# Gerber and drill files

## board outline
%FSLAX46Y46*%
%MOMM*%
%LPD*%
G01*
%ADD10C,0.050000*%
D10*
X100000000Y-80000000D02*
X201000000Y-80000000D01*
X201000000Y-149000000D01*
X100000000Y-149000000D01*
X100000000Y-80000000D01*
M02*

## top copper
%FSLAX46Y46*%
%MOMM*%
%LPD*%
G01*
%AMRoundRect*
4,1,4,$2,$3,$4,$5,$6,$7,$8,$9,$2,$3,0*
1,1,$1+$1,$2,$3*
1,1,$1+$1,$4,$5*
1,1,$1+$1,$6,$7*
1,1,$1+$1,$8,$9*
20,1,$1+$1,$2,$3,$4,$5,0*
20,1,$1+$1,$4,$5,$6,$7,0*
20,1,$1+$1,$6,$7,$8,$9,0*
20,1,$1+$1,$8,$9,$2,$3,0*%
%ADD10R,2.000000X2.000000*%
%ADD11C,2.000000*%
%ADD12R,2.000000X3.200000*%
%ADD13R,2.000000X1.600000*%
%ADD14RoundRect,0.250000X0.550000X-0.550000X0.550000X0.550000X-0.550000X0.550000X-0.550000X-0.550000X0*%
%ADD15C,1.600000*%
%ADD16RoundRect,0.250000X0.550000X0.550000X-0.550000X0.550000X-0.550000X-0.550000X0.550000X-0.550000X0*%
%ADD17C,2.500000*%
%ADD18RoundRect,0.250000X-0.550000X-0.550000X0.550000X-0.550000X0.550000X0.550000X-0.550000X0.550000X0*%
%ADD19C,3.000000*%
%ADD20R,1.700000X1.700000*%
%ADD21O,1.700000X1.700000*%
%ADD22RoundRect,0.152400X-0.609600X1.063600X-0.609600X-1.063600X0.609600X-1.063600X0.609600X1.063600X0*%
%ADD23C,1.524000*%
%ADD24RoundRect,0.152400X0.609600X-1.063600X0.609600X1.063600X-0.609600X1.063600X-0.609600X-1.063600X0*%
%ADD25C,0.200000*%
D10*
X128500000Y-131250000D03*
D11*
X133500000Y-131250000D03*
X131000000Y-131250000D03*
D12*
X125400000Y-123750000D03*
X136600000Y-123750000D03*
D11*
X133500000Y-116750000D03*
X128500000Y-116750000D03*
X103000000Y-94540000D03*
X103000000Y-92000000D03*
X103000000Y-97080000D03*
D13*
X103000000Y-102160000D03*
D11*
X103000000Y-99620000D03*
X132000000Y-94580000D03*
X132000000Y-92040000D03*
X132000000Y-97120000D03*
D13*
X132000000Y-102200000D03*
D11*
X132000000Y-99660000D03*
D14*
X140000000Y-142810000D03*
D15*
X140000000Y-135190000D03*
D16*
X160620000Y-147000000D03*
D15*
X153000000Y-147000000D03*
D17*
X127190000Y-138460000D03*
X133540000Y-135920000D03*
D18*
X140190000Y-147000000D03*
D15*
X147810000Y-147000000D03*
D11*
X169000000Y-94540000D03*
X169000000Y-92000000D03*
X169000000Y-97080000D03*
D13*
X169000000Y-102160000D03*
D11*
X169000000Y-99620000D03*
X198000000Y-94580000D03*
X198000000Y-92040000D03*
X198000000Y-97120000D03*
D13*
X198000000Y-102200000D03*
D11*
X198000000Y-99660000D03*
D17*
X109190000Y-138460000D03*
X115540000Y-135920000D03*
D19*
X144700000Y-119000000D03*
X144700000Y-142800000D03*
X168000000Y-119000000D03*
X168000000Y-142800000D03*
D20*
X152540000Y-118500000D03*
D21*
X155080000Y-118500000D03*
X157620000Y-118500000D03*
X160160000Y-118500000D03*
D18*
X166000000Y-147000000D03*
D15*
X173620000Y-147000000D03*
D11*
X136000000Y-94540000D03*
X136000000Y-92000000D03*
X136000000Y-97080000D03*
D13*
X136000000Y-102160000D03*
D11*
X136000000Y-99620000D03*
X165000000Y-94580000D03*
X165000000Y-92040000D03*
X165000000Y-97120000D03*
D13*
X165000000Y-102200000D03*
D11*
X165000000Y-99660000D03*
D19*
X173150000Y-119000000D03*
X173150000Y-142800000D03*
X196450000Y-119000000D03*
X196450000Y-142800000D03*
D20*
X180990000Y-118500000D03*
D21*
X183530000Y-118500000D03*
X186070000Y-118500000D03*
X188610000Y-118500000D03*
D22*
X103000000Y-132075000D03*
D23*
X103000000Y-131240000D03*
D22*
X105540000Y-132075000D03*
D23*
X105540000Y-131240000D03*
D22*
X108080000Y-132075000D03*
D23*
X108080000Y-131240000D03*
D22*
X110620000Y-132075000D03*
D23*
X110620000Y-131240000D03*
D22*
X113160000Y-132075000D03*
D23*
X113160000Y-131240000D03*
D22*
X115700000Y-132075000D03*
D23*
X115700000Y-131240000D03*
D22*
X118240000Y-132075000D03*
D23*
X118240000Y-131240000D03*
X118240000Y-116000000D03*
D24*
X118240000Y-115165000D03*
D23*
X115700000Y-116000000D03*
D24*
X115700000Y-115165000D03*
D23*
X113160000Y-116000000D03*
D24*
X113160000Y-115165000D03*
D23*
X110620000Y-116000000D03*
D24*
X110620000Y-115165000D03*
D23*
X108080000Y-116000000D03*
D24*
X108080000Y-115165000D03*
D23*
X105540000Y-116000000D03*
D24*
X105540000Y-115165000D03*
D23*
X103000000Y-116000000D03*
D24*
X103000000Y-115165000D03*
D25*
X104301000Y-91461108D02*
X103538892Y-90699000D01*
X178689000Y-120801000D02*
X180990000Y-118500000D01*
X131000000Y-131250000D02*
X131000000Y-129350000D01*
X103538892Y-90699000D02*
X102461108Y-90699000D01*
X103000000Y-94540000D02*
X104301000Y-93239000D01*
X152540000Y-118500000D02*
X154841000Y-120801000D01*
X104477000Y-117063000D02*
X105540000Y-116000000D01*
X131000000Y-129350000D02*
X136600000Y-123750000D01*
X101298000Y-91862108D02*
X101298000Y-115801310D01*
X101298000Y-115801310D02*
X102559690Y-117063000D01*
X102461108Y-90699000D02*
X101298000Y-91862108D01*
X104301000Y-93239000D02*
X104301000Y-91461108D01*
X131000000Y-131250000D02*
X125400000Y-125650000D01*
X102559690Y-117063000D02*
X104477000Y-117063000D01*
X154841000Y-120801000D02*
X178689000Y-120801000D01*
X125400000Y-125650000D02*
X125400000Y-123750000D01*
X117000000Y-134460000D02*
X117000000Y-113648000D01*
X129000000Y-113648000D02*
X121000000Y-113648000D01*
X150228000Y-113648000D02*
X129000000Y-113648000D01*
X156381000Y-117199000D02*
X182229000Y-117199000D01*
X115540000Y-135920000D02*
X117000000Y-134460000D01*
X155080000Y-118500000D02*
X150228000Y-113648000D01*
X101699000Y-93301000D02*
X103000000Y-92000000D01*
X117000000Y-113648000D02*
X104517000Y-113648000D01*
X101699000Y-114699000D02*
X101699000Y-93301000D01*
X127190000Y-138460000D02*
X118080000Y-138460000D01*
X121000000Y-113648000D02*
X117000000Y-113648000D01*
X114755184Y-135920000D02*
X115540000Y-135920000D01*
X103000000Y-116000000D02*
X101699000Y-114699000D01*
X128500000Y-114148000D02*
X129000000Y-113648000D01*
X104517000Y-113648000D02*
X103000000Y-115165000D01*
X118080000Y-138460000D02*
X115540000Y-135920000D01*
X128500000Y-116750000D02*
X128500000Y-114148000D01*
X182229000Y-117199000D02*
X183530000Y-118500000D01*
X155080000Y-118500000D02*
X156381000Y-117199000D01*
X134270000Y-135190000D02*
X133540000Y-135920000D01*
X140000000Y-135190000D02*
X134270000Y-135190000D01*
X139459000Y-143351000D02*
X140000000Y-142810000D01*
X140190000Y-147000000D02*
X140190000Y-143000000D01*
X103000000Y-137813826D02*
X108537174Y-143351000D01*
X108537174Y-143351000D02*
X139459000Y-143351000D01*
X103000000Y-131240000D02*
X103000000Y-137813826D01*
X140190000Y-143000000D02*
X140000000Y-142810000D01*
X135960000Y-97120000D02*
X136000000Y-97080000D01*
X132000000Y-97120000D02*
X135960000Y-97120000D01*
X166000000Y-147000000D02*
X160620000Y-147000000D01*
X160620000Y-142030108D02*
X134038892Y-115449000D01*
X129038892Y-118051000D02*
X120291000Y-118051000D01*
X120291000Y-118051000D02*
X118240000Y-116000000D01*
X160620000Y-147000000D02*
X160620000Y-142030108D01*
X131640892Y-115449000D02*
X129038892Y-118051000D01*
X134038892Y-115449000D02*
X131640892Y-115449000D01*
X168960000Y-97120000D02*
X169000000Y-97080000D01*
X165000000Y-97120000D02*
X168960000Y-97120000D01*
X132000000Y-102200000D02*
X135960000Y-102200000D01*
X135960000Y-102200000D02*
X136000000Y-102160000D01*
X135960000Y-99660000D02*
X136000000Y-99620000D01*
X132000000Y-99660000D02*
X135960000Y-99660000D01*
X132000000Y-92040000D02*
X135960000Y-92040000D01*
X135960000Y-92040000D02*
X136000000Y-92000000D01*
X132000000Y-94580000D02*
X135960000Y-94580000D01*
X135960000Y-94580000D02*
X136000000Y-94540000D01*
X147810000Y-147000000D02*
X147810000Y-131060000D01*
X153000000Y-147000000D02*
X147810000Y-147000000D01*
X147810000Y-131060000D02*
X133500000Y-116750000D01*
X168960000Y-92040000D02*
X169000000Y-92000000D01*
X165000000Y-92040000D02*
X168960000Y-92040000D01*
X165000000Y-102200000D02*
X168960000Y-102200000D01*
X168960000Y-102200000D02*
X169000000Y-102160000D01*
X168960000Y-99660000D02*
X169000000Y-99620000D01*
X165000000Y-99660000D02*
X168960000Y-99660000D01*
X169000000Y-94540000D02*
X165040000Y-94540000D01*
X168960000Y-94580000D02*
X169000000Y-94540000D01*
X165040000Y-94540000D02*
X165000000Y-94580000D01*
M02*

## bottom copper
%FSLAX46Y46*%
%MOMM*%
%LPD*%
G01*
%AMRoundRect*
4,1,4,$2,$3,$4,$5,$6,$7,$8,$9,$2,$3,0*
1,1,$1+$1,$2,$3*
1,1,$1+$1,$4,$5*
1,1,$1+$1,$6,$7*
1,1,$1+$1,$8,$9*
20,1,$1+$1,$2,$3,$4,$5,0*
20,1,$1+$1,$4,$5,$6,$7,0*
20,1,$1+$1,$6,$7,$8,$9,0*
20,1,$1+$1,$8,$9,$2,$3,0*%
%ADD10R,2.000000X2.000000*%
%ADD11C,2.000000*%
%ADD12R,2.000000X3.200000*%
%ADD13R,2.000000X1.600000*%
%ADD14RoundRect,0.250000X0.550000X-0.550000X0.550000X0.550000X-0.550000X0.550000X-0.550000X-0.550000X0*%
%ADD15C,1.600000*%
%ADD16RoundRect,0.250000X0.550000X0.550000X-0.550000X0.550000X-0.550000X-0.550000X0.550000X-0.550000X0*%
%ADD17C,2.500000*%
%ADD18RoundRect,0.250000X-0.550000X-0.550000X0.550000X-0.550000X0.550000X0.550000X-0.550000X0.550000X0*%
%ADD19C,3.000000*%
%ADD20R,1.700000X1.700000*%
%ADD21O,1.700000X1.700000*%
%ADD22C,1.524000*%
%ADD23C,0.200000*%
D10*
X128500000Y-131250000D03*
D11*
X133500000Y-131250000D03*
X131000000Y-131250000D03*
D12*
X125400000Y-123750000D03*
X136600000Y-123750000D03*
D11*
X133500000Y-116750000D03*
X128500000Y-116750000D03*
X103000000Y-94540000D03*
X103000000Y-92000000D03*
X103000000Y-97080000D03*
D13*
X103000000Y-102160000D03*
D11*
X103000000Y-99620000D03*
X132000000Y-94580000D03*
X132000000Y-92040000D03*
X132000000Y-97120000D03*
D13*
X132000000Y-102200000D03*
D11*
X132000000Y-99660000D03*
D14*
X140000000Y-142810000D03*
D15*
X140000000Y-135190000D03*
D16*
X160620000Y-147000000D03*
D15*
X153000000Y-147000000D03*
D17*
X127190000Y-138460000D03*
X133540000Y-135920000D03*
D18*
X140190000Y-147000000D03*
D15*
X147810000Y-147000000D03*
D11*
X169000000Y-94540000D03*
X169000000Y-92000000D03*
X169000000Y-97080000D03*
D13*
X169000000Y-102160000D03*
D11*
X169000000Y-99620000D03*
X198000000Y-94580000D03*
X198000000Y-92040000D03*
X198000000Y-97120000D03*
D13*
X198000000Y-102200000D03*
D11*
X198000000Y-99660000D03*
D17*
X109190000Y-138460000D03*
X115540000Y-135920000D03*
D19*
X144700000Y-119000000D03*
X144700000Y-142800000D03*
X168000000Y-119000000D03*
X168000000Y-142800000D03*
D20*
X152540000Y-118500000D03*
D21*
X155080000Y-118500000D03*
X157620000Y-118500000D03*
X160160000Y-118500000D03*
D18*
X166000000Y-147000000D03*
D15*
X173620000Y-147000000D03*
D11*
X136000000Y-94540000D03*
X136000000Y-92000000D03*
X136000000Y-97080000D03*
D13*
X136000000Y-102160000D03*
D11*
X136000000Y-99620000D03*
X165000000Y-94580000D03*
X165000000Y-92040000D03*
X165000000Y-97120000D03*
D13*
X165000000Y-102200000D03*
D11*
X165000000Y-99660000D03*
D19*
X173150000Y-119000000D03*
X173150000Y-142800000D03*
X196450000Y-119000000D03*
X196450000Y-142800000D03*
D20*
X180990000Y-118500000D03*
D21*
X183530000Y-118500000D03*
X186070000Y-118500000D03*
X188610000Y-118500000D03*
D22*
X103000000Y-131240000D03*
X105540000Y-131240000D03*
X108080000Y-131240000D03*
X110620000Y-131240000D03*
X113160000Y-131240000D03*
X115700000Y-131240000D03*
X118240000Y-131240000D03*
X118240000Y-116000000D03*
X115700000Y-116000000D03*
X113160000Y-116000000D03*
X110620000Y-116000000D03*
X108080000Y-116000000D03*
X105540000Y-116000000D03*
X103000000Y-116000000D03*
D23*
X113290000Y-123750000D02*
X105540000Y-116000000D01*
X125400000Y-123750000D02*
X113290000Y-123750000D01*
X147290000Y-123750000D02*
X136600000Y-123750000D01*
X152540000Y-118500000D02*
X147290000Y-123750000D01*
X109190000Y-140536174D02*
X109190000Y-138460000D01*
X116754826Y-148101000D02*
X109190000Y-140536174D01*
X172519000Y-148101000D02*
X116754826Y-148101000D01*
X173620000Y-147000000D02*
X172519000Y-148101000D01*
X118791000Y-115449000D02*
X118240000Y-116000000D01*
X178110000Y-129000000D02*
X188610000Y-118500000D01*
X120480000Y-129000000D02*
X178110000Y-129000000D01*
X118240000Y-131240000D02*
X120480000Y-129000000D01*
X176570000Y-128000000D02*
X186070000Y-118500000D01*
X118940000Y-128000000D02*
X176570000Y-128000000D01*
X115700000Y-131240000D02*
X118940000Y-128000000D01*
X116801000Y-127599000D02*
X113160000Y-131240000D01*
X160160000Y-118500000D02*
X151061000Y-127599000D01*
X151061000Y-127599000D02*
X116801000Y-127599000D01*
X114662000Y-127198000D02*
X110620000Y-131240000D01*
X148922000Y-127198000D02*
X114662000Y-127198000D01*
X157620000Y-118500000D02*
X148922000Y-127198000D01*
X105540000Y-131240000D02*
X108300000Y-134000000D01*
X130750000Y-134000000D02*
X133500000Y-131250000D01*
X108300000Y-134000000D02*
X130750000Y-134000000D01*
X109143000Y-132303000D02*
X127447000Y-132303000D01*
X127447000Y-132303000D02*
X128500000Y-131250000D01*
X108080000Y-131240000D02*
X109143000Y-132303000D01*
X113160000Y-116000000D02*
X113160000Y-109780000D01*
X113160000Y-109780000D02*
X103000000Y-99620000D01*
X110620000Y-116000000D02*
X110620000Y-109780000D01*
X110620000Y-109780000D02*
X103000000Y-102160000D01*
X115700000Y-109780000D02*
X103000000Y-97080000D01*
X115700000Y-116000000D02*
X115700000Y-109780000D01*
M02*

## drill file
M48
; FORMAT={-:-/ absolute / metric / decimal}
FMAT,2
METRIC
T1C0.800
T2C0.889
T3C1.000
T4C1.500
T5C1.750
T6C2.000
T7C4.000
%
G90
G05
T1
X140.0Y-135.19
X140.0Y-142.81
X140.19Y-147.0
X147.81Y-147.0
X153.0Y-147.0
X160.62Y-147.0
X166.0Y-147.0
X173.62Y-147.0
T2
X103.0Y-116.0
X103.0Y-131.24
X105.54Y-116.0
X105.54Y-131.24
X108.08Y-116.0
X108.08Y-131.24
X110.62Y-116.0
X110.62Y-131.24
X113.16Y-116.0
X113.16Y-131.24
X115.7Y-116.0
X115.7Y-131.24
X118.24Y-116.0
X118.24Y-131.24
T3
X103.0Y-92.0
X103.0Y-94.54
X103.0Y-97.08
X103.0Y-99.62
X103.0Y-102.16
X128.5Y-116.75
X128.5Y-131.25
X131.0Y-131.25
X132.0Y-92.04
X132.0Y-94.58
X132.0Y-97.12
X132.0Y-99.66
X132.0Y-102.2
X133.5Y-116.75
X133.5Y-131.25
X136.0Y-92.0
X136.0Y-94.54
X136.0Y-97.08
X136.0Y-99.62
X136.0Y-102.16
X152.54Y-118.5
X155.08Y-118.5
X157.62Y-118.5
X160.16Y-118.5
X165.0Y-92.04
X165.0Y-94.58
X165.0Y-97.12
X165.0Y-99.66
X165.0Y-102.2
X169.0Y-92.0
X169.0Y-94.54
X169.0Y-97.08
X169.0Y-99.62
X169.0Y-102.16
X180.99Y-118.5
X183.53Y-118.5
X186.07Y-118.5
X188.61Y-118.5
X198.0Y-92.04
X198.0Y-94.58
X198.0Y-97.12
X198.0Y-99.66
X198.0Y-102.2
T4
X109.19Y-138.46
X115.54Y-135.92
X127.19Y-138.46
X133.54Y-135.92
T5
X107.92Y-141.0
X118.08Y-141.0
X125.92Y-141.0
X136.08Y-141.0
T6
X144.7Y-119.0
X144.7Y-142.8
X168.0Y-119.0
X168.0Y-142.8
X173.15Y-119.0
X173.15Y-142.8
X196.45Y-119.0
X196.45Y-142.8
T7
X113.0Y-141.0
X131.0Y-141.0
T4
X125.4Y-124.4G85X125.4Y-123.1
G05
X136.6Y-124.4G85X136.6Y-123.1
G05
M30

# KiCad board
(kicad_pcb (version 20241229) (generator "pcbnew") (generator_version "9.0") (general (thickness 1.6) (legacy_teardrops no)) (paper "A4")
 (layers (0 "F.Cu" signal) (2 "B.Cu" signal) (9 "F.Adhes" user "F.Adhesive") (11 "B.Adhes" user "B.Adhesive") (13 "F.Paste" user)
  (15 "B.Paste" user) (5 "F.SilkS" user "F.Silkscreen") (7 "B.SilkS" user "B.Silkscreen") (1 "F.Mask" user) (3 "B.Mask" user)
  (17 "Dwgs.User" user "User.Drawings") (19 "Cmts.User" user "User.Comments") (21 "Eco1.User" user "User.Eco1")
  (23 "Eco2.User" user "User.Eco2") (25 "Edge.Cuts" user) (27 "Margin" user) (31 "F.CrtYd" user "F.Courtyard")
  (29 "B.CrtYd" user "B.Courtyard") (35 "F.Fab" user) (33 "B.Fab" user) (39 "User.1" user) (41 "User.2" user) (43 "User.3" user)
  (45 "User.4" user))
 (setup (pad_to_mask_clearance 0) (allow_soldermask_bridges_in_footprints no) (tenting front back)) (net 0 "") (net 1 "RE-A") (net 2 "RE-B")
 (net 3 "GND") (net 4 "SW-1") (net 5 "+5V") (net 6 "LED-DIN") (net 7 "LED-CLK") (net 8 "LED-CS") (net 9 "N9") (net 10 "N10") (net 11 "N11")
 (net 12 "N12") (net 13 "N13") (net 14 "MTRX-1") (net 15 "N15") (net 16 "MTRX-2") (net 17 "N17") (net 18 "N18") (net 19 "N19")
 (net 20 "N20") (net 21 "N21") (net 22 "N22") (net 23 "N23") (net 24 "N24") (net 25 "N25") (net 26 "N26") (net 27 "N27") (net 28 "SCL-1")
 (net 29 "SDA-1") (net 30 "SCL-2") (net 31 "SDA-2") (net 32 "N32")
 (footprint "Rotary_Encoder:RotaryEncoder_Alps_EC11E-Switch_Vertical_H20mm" (layer "F.Cu") (at 128.5 131.25 90)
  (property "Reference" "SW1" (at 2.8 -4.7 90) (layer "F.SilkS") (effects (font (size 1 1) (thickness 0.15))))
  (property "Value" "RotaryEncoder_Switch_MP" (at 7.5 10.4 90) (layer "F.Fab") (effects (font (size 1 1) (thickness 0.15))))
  (pad "A" thru_hole rect (at 0 0 90) (size 2 2) (drill 1) (layers "*.Cu" "*.Mask") (remove_unused_layers no) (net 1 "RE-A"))
  (pad "B" thru_hole circle (at 0 5 90) (size 2 2) (drill 1) (layers "*.Cu" "*.Mask") (remove_unused_layers no) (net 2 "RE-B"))
  (pad "C" thru_hole circle (at 0 2.5 90) (size 2 2) (drill 1) (layers "*.Cu" "*.Mask") (remove_unused_layers no) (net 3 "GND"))
  (pad "MP" thru_hole rect (at 7.5 -3.1 90) (size 3.2 2) (drill oval 2.8 1.5) (layers "*.Cu" "*.Mask") (remove_unused_layers no)
   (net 3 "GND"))
  (pad "MP" thru_hole rect (at 7.5 8.1 90) (size 3.2 2) (drill oval 2.8 1.5) (layers "*.Cu" "*.Mask") (remove_unused_layers no)
   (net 3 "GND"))
  (pad "S1" thru_hole circle (at 14.5 5 90) (size 2 2) (drill 1) (layers "*.Cu" "*.Mask") (remove_unused_layers no) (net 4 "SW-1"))
  (pad "S2" thru_hole circle (at 14.5 0 90) (size 2 2) (drill 1) (layers "*.Cu" "*.Mask") (remove_unused_layers no) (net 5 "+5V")))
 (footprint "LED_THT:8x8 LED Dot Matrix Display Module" (layer "F.Cu") (at 118 97.04)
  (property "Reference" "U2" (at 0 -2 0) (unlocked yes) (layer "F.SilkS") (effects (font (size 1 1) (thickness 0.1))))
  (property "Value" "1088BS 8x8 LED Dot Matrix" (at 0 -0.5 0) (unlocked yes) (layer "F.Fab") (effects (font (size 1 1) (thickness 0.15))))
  (pad "1" thru_hole circle (at -15 -2.5) (size 2 2) (drill 1) (layers "*.Cu" "*.Mask") (remove_unused_layers no) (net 3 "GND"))
  (pad "2" thru_hole circle (at -15 -5.04) (size 2 2) (drill 1) (layers "*.Cu" "*.Mask") (remove_unused_layers no) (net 5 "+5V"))
  (pad "3" thru_hole circle (at -15 0.04) (size 2 2) (drill 1) (layers "*.Cu" "*.Mask") (remove_unused_layers no) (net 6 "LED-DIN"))
  (pad "4" thru_hole rect (at -15 5.12) (size 2 1.6) (drill 1) (layers "*.Cu" "*.Mask") (remove_unused_layers no) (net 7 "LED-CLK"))
  (pad "5" thru_hole circle (at -15 2.58) (size 2 2) (drill 1) (layers "*.Cu" "*.Mask") (remove_unused_layers no) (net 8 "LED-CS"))
  (pad "6" thru_hole circle (at 14 -2.46) (size 2 2) (drill 1) (layers "*.Cu" "*.Mask") (remove_unused_layers no) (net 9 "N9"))
  (pad "7" thru_hole circle (at 14 -5) (size 2 2) (drill 1) (layers "*.Cu" "*.Mask") (remove_unused_layers no) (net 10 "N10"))
  (pad "8" thru_hole circle (at 14 0.08) (size 2 2) (drill 1) (layers "*.Cu" "*.Mask") (remove_unused_layers no) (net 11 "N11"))
  (pad "9" thru_hole rect (at 14 5.16) (size 2 1.6) (drill 1) (layers "*.Cu" "*.Mask") (remove_unused_layers no) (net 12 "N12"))
  (pad "10" thru_hole circle (at 14 2.62) (size 2 2) (drill 1) (layers "*.Cu" "*.Mask") (remove_unused_layers no) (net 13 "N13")))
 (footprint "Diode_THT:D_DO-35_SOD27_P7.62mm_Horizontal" (layer "F.Cu") (at 140 142.81 90)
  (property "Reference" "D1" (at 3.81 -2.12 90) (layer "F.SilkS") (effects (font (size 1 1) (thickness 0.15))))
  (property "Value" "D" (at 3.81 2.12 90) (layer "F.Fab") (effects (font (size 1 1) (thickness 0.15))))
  (pad "1" thru_hole roundrect (at 0 0 90) (size 1.6 1.6) (drill 0.8) (layers "*.Cu" "*.Mask") (remove_unused_layers no)
   (roundrect_rratio 0.15625) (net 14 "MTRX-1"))
  (pad "2" thru_hole circle (at 7.62 0 90) (size 1.6 1.6) (drill 0.8) (layers "*.Cu" "*.Mask") (remove_unused_layers no) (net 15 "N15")))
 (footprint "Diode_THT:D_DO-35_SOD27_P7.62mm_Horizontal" (layer "F.Cu") (at 160.62 147 180)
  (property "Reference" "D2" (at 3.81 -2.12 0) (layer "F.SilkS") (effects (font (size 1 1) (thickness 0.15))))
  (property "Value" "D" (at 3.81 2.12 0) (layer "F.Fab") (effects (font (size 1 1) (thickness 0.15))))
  (pad "1" thru_hole roundrect (at 0 0 180) (size 1.6 1.6) (drill 0.8) (layers "*.Cu" "*.Mask") (remove_unused_layers no)
   (roundrect_rratio 0.15625) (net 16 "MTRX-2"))
  (pad "2" thru_hole circle (at 7.62 0 180) (size 1.6 1.6) (drill 0.8) (layers "*.Cu" "*.Mask") (remove_unused_layers no) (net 4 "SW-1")))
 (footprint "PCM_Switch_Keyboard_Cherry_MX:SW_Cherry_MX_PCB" (layer "F.Cu") (at 131 141)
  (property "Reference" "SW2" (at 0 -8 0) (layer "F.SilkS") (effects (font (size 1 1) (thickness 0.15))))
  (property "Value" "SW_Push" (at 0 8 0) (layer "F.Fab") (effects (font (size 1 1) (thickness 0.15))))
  (pad "" np_thru_hole circle (at -5.08 0) (size 1.75 1.75) (drill 1.75) (layers "*.Cu" "*.Mask"))
  (pad "" np_thru_hole circle (at 0 0) (size 4 4) (drill 4) (layers "*.Cu" "*.Mask"))
  (pad "" np_thru_hole circle (at 5.08 0) (size 1.75 1.75) (drill 1.75) (layers "*.Cu" "*.Mask"))
  (pad "1" thru_hole circle (at -3.81 -2.54) (size 2.5 2.5) (drill 1.5) (layers "*.Cu" "*.Mask") (remove_unused_layers no) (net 5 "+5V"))
  (pad "2" thru_hole circle (at 2.54 -5.08) (size 2.5 2.5) (drill 1.5) (layers "*.Cu" "*.Mask") (remove_unused_layers no) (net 15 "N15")))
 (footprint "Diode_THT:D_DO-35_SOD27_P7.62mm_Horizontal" (layer "F.Cu") (at 140.19 147)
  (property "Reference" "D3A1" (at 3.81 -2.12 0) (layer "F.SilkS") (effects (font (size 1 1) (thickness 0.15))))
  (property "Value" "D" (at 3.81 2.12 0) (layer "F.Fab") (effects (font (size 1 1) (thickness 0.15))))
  (pad "1" thru_hole roundrect (at 0 0) (size 1.6 1.6) (drill 0.8) (layers "*.Cu" "*.Mask") (remove_unused_layers no)
   (roundrect_rratio 0.15625) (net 14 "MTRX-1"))
  (pad "2" thru_hole circle (at 7.62 0) (size 1.6 1.6) (drill 0.8) (layers "*.Cu" "*.Mask") (remove_unused_layers no) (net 4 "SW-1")))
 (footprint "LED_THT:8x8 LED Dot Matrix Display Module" (layer "F.Cu") (at 184 97.04)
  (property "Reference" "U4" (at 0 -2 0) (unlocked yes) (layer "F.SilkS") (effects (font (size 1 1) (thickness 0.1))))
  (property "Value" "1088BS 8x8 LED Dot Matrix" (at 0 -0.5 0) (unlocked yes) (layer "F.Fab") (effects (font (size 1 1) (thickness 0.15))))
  (pad "1" thru_hole circle (at -15 -2.5) (size 2 2) (drill 1) (layers "*.Cu" "*.Mask") (remove_unused_layers no) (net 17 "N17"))
  (pad "2" thru_hole circle (at -15 -5.04) (size 2 2) (drill 1) (layers "*.Cu" "*.Mask") (remove_unused_layers no) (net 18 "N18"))
  (pad "3" thru_hole circle (at -15 0.04) (size 2 2) (drill 1) (layers "*.Cu" "*.Mask") (remove_unused_layers no) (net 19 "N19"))
  (pad "4" thru_hole rect (at -15 5.12) (size 2 1.6) (drill 1) (layers "*.Cu" "*.Mask") (remove_unused_layers no) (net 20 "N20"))
  (pad "5" thru_hole circle (at -15 2.58) (size 2 2) (drill 1) (layers "*.Cu" "*.Mask") (remove_unused_layers no) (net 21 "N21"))
  (pad "6" thru_hole circle (at 14 -2.46) (size 2 2) (drill 1) (layers "*.Cu" "*.Mask") (remove_unused_layers no) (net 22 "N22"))
  (pad "7" thru_hole circle (at 14 -5) (size 2 2) (drill 1) (layers "*.Cu" "*.Mask") (remove_unused_layers no) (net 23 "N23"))
  (pad "8" thru_hole circle (at 14 0.08) (size 2 2) (drill 1) (layers "*.Cu" "*.Mask") (remove_unused_layers no) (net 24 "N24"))
  (pad "9" thru_hole rect (at 14 5.16) (size 2 1.6) (drill 1) (layers "*.Cu" "*.Mask") (remove_unused_layers no) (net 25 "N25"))
  (pad "10" thru_hole circle (at 14 2.62) (size 2 2) (drill 1) (layers "*.Cu" "*.Mask") (remove_unused_layers no) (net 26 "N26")))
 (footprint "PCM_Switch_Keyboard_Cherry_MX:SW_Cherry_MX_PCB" (layer "F.Cu") (at 113 141)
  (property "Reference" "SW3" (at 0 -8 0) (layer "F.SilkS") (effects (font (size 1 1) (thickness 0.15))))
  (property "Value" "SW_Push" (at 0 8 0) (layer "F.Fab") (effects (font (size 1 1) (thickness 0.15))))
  (pad "" np_thru_hole circle (at -5.08 0) (size 1.75 1.75) (drill 1.75) (layers "*.Cu" "*.Mask"))
  (pad "" np_thru_hole circle (at 0 0) (size 4 4) (drill 4) (layers "*.Cu" "*.Mask"))
  (pad "" np_thru_hole circle (at 5.08 0) (size 1.75 1.75) (drill 1.75) (layers "*.Cu" "*.Mask"))
  (pad "1" thru_hole circle (at -3.81 -2.54) (size 2.5 2.5) (drill 1.5) (layers "*.Cu" "*.Mask") (remove_unused_layers no) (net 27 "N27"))
  (pad "2" thru_hole circle (at 2.54 -5.08) (size 2.5 2.5) (drill 1.5) (layers "*.Cu" "*.Mask") (remove_unused_layers no) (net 5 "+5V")))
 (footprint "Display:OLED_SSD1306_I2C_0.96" (layer "F.Cu") (at 152.54 118.5)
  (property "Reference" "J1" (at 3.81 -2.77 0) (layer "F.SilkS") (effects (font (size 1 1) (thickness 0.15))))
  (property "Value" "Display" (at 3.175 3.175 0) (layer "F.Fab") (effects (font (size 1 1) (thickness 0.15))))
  (pad "" np_thru_hole circle (at -7.84 0.5) (size 3 3) (drill 2) (layers "*.Cu" "*.Mask"))
  (pad "" np_thru_hole circle (at -7.84 24.3) (size 3 3) (drill 2) (layers "*.Cu" "*.Mask"))
  (pad "" np_thru_hole circle (at 15.46 0.5) (size 3 3) (drill 2) (layers "*.Cu" "*.Mask"))
  (pad "" np_thru_hole circle (at 15.46 24.3) (size 3 3) (drill 2) (layers "*.Cu" "*.Mask"))
  (pad "1" thru_hole rect (at 0 0 90) (size 1.7 1.7) (drill 1) (layers "*.Cu" "*.Mask") (remove_unused_layers no) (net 3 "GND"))
  (pad "2" thru_hole oval (at 2.54 0 90) (size 1.7 1.7) (drill 1) (layers "*.Cu" "*.Mask") (remove_unused_layers no) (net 5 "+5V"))
  (pad "3" thru_hole oval (at 5.08 0 90) (size 1.7 1.7) (drill 1) (layers "*.Cu" "*.Mask") (remove_unused_layers no) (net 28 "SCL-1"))
  (pad "4" thru_hole oval (at 7.62 0 90) (size 1.7 1.7) (drill 1) (layers "*.Cu" "*.Mask") (remove_unused_layers no) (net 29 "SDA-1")))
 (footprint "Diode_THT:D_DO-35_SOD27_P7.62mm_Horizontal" (layer "F.Cu") (at 166 147)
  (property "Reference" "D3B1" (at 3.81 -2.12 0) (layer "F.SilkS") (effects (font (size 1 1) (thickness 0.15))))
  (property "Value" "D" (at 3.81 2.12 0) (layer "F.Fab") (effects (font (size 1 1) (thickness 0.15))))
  (pad "1" thru_hole roundrect (at 0 0) (size 1.6 1.6) (drill 0.8) (layers "*.Cu" "*.Mask") (remove_unused_layers no)
   (roundrect_rratio 0.15625) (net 16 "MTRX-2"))
  (pad "2" thru_hole circle (at 7.62 0) (size 1.6 1.6) (drill 0.8) (layers "*.Cu" "*.Mask") (remove_unused_layers no) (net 27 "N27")))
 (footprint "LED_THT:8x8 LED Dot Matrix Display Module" (layer "F.Cu") (at 151 97.04)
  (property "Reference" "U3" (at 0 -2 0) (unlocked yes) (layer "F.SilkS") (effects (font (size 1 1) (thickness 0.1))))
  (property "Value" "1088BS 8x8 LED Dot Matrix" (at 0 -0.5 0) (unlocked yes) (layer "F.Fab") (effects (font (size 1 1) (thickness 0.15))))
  (pad "1" thru_hole circle (at -15 -2.5) (size 2 2) (drill 1) (layers "*.Cu" "*.Mask") (remove_unused_layers no) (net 9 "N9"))
  (pad "2" thru_hole circle (at -15 -5.04) (size 2 2) (drill 1) (layers "*.Cu" "*.Mask") (remove_unused_layers no) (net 10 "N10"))
  (pad "3" thru_hole circle (at -15 0.04) (size 2 2) (drill 1) (layers "*.Cu" "*.Mask") (remove_unused_layers no) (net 11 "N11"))
  (pad "4" thru_hole rect (at -15 5.12) (size 2 1.6) (drill 1) (layers "*.Cu" "*.Mask") (remove_unused_layers no) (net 12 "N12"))
  (pad "5" thru_hole circle (at -15 2.58) (size 2 2) (drill 1) (layers "*.Cu" "*.Mask") (remove_unused_layers no) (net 13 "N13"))
  (pad "6" thru_hole circle (at 14 -2.46) (size 2 2) (drill 1) (layers "*.Cu" "*.Mask") (remove_unused_layers no) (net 17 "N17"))
  (pad "7" thru_hole circle (at 14 -5) (size 2 2) (drill 1) (layers "*.Cu" "*.Mask") (remove_unused_layers no) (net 18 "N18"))
  (pad "8" thru_hole circle (at 14 0.08) (size 2 2) (drill 1) (layers "*.Cu" "*.Mask") (remove_unused_layers no) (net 19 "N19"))
  (pad "9" thru_hole rect (at 14 5.16) (size 2 1.6) (drill 1) (layers "*.Cu" "*.Mask") (remove_unused_layers no) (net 20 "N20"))
  (pad "10" thru_hole circle (at 14 2.62) (size 2 2) (drill 1) (layers "*.Cu" "*.Mask") (remove_unused_layers no) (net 21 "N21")))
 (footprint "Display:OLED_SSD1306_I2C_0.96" (layer "F.Cu") (at 180.99 118.5)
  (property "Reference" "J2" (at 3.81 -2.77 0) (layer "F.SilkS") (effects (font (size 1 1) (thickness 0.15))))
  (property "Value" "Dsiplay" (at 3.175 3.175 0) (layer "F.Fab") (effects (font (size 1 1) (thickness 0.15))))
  (pad "" np_thru_hole circle (at -7.84 0.5) (size 3 3) (drill 2) (layers "*.Cu" "*.Mask"))
  (pad "" np_thru_hole circle (at -7.84 24.3) (size 3 3) (drill 2) (layers "*.Cu" "*.Mask"))
  (pad "" np_thru_hole circle (at 15.46 0.5) (size 3 3) (drill 2) (layers "*.Cu" "*.Mask"))
  (pad "" np_thru_hole circle (at 15.46 24.3) (size 3 3) (drill 2) (layers "*.Cu" "*.Mask"))
  (pad "1" thru_hole rect (at 0 0 90) (size 1.7 1.7) (drill 1) (layers "*.Cu" "*.Mask") (remove_unused_layers no) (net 3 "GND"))
  (pad "2" thru_hole oval (at 2.54 0 90) (size 1.7 1.7) (drill 1) (layers "*.Cu" "*.Mask") (remove_unused_layers no) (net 5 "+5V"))
  (pad "3" thru_hole oval (at 5.08 0 90) (size 1.7 1.7) (drill 1) (layers "*.Cu" "*.Mask") (remove_unused_layers no) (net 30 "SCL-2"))
  (pad "4" thru_hole oval (at 7.62 0 90) (size 1.7 1.7) (drill 1) (layers "*.Cu" "*.Mask") (remove_unused_layers no) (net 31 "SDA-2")))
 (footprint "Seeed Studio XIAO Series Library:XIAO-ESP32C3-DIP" (layer "F.Cu") (at 110.62 123.5 90)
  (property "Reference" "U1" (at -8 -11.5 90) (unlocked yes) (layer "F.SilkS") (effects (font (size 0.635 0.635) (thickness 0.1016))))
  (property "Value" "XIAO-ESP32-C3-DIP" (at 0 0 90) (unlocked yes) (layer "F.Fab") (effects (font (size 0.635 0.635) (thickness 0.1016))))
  (pad "1" smd roundrect (at -8.575 -7.62 270) (size 2.432 1.524) (layers "F.Cu" "F.Mask") (roundrect_rratio 0.1) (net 14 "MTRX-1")
   (thermal_bridge_angle 45))
  (pad "1" thru_hole circle (at -7.74 -7.62 270) (size 1.524 1.524) (drill 0.889) (layers "*.Cu" "*.Mask") (remove_unused_layers no)
   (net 14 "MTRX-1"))
  (pad "2" smd roundrect (at -8.575 -5.08 270) (size 2.432 1.524) (layers "F.Cu" "F.Mask") (roundrect_rratio 0.1) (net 2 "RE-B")
   (thermal_bridge_angle 45))
  (pad "2" thru_hole circle (at -7.74 -5.08 270) (size 1.524 1.524) (drill 0.889) (layers "*.Cu" "*.Mask") (remove_unused_layers no)
   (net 2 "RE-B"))
  (pad "3" smd roundrect (at -8.575 -2.54 270) (size 2.432 1.524) (layers "F.Cu" "F.Mask") (roundrect_rratio 0.1) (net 1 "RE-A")
   (thermal_bridge_angle 45))
  (pad "3" thru_hole circle (at -7.74 -2.54 270) (size 1.524 1.524) (drill 0.889) (layers "*.Cu" "*.Mask") (remove_unused_layers no)
   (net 1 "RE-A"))
  (pad "4" smd roundrect (at -8.575 0 270) (size 2.432 1.524) (layers "F.Cu" "F.Mask") (roundrect_rratio 0.1) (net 28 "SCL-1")
   (thermal_bridge_angle 45))
  (pad "4" thru_hole circle (at -7.74 0 270) (size 1.524 1.524) (drill 0.889) (layers "*.Cu" "*.Mask") (remove_unused_layers no)
   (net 28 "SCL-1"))
  (pad "5" smd roundrect (at -8.575 2.54 270) (size 2.432 1.524) (layers "F.Cu" "F.Mask") (roundrect_rratio 0.1) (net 29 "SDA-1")
   (thermal_bridge_angle 45))
  (pad "5" thru_hole circle (at -7.74 2.54 270) (size 1.524 1.524) (drill 0.889) (layers "*.Cu" "*.Mask") (remove_unused_layers no)
   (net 29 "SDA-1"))
  (pad "6" smd roundrect (at -8.575 5.08 270) (size 2.432 1.524) (layers "F.Cu" "F.Mask") (roundrect_rratio 0.1) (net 30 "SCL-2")
   (thermal_bridge_angle 45))
  (pad "6" thru_hole circle (at -7.74 5.08 270) (size 1.524 1.524) (drill 0.889) (layers "*.Cu" "*.Mask") (remove_unused_layers no)
   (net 30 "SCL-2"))
  (pad "7" smd roundrect (at -8.575 7.62 270) (size 2.432 1.524) (layers "F.Cu" "F.Mask") (roundrect_rratio 0.1) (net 31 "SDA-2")
   (thermal_bridge_angle 45))
  (pad "7" thru_hole circle (at -7.74 7.62 270) (size 1.524 1.524) (drill 0.889) (layers "*.Cu" "*.Mask") (remove_unused_layers no)
   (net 31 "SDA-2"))
  (pad "8" thru_hole circle (at 7.5 7.62 90) (size 1.524 1.524) (drill 0.889) (layers "*.Cu" "*.Mask") (remove_unused_layers no)
   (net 16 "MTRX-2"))
  (pad "8" smd roundrect (at 8.335 7.62 90) (size 2.432 1.524) (layers "F.Cu" "F.Mask") (roundrect_rratio 0.1) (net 16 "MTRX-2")
   (thermal_bridge_angle 45))
  (pad "9" thru_hole circle (at 7.5 5.08 90) (size 1.524 1.524) (drill 0.889) (layers "*.Cu" "*.Mask") (remove_unused_layers no)
   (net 6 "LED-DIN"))
  (pad "9" smd roundrect (at 8.335 5.08 90) (size 2.432 1.524) (layers "F.Cu" "F.Mask") (roundrect_rratio 0.1) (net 6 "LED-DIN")
   (thermal_bridge_angle 45))
  (pad "10" thru_hole circle (at 7.5 2.54 90) (size 1.524 1.524) (drill 0.889) (layers "*.Cu" "*.Mask") (remove_unused_layers no)
   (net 8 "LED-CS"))
  (pad "10" smd roundrect (at 8.335 2.54 90) (size 2.432 1.524) (layers "F.Cu" "F.Mask") (roundrect_rratio 0.1) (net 8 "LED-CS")
   (thermal_bridge_angle 45))
  (pad "11" thru_hole circle (at 7.5 0 90) (size 1.524 1.524) (drill 0.889) (layers "*.Cu" "*.Mask") (remove_unused_layers no)
   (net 7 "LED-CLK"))
  (pad "11" smd roundrect (at 8.335 0 90) (size 2.432 1.524) (layers "F.Cu" "F.Mask") (roundrect_rratio 0.1) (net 7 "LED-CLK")
   (thermal_bridge_angle 45))
  (pad "12" thru_hole circle (at 7.5 -2.54 90) (size 1.524 1.524) (drill 0.889) (layers "*.Cu" "*.Mask") (remove_unused_layers no)
   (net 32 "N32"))
  (pad "12" smd roundrect (at 8.335 -2.54 90) (size 2.432 1.524) (layers "F.Cu" "F.Mask") (roundrect_rratio 0.1) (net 32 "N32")
   (thermal_bridge_angle 45))
  (pad "13" thru_hole circle (at 7.5 -5.08 90) (size 1.524 1.524) (drill 0.889) (layers "*.Cu" "*.Mask") (remove_unused_layers no)
   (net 3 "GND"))
  (pad "13" smd roundrect (at 8.335 -5.08 90) (size 2.432 1.524) (layers "F.Cu" "F.Mask") (roundrect_rratio 0.1) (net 3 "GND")
   (thermal_bridge_angle 45))
  (pad "14" thru_hole circle (at 7.5 -7.62 90) (size 1.524 1.524) (drill 0.889) (layers "*.Cu" "*.Mask") (remove_unused_layers no)
   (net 5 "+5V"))
  (pad "14" smd roundrect (at 8.335 -7.62 90) (size 2.432 1.524) (layers "F.Cu" "F.Mask") (roundrect_rratio 0.1) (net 5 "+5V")
   (thermal_bridge_angle 45)))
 (gr_rect (start 100 80) (end 201 149) (stroke (width 0.05) (type default)) (fill no) (layer "Edge.Cuts"))
 (segment (start 104.301 91.461108) (end 103.538892 90.699) (width 0.2) (layer "F.Cu") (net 3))
 (segment (start 178.689 120.801) (end 180.99 118.5) (width 0.2) (layer "F.Cu") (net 3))
 (segment (start 131 131.25) (end 131 129.35) (width 0.2) (layer "F.Cu") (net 3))
 (segment (start 103.538892 90.699) (end 102.461108 90.699) (width 0.2) (layer "F.Cu") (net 3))
 (segment (start 103 94.54) (end 104.301 93.239) (width 0.2) (layer "F.Cu") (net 3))
 (segment (start 152.54 118.5) (end 154.841 120.801) (width 0.2) (layer "F.Cu") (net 3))
 (segment (start 104.477 117.063) (end 105.54 116) (width 0.2) (layer "F.Cu") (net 3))
 (segment (start 131 129.35) (end 136.6 123.75) (width 0.2) (layer "F.Cu") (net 3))
 (segment (start 101.298 91.862108) (end 101.298 115.80131) (width 0.2) (layer "F.Cu") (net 3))
 (segment (start 101.298 115.80131) (end 102.55969 117.063) (width 0.2) (layer "F.Cu") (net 3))
 (segment (start 102.461108 90.699) (end 101.298 91.862108) (width 0.2) (layer "F.Cu") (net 3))
 (segment (start 104.301 93.239) (end 104.301 91.461108) (width 0.2) (layer "F.Cu") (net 3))
 (segment (start 131 131.25) (end 125.4 125.65) (width 0.2) (layer "F.Cu") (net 3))
 (segment (start 102.55969 117.063) (end 104.477 117.063) (width 0.2) (layer "F.Cu") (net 3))
 (segment (start 154.841 120.801) (end 178.689 120.801) (width 0.2) (layer "F.Cu") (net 3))
 (segment (start 125.4 125.65) (end 125.4 123.75) (width 0.2) (layer "F.Cu") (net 3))
 (segment (start 113.29 123.75) (end 105.54 116) (width 0.2) (layer "B.Cu") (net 3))
 (segment (start 125.4 123.75) (end 113.29 123.75) (width 0.2) (layer "B.Cu") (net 3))
 (segment (start 147.29 123.75) (end 136.6 123.75) (width 0.2) (layer "B.Cu") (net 3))
 (segment (start 152.54 118.5) (end 147.29 123.75) (width 0.2) (layer "B.Cu") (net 3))
 (segment (start 117 134.46) (end 117 113.648) (width 0.2) (layer "F.Cu") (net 5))
 (segment (start 129 113.648) (end 121 113.648) (width 0.2) (layer "F.Cu") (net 5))
 (segment (start 150.228 113.648) (end 129 113.648) (width 0.2) (layer "F.Cu") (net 5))
 (segment (start 156.381 117.199) (end 182.229 117.199) (width 0.2) (layer "F.Cu") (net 5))
 (segment (start 115.54 135.92) (end 117 134.46) (width 0.2) (layer "F.Cu") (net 5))
 (segment (start 155.08 118.5) (end 150.228 113.648) (width 0.2) (layer "F.Cu") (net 5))
 (segment (start 101.699 93.301) (end 103 92) (width 0.2) (layer "F.Cu") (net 5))
 (segment (start 117 113.648) (end 104.517 113.648) (width 0.2) (layer "F.Cu") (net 5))
 (segment (start 101.699 114.699) (end 101.699 93.301) (width 0.2) (layer "F.Cu") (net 5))
 (segment (start 127.19 138.46) (end 118.08 138.46) (width 0.2) (layer "F.Cu") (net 5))
 (segment (start 121 113.648) (end 117 113.648) (width 0.2) (layer "F.Cu") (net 5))
 (segment (start 114.755184 135.92) (end 115.54 135.92) (width 0.2) (layer "F.Cu") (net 5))
 (segment (start 103 116) (end 101.699 114.699) (width 0.2) (layer "F.Cu") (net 5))
 (segment (start 128.5 114.148) (end 129 113.648) (width 0.2) (layer "F.Cu") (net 5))
 (segment (start 104.517 113.648) (end 103 115.165) (width 0.2) (layer "F.Cu") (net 5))
 (segment (start 118.08 138.46) (end 115.54 135.92) (width 0.2) (layer "F.Cu") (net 5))
 (segment (start 128.5 116.75) (end 128.5 114.148) (width 0.2) (layer "F.Cu") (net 5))
 (segment (start 182.229 117.199) (end 183.53 118.5) (width 0.2) (layer "F.Cu") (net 5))
 (segment (start 155.08 118.5) (end 156.381 117.199) (width 0.2) (layer "F.Cu") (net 5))
 (segment (start 134.27 135.19) (end 133.54 135.92) (width 0.2) (layer "F.Cu") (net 15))
 (segment (start 140 135.19) (end 134.27 135.19) (width 0.2) (layer "F.Cu") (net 15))
 (segment (start 109.19 140.536174) (end 109.19 138.46) (width 0.2) (layer "B.Cu") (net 27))
 (segment (start 116.754826 148.101) (end 109.19 140.536174) (width 0.2) (layer "B.Cu") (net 27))
 (segment (start 172.519 148.101) (end 116.754826 148.101) (width 0.2) (layer "B.Cu") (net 27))
 (segment (start 173.62 147) (end 172.519 148.101) (width 0.2) (layer "B.Cu") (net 27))
 (segment (start 139.459 143.351) (end 140 142.81) (width 0.2) (layer "F.Cu") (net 14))
 (segment (start 140.19 147) (end 140.19 143) (width 0.2) (layer "F.Cu") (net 14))
 (segment (start 103 137.813826) (end 108.537174 143.351) (width 0.2) (layer "F.Cu") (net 14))
 (segment (start 108.537174 143.351) (end 139.459 143.351) (width 0.2) (layer "F.Cu") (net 14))
 (segment (start 103 131.24) (end 103 137.813826) (width 0.2) (layer "F.Cu") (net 14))
 (segment (start 140.19 143) (end 140 142.81) (width 0.2) (layer "F.Cu") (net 14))
 (segment (start 135.96 97.12) (end 136 97.08) (width 0.2) (layer "F.Cu") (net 11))
 (segment (start 132 97.12) (end 135.96 97.12) (width 0.2) (layer "F.Cu") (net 11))
 (segment (start 166 147) (end 160.62 147) (width 0.2) (layer "F.Cu") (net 16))
 (segment (start 160.62 142.030108) (end 134.038892 115.449) (width 0.2) (layer "F.Cu") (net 16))
 (segment (start 129.038892 118.051) (end 120.291 118.051) (width 0.2) (layer "F.Cu") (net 16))
 (segment (start 120.291 118.051) (end 118.24 116) (width 0.2) (layer "F.Cu") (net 16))
 (segment (start 160.62 147) (end 160.62 142.030108) (width 0.2) (layer "F.Cu") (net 16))
 (segment (start 131.640892 115.449) (end 129.038892 118.051) (width 0.2) (layer "F.Cu") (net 16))
 (segment (start 134.038892 115.449) (end 131.640892 115.449) (width 0.2) (layer "F.Cu") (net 16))
 (segment (start 118.791 115.449) (end 118.24 116) (width 0.2) (layer "B.Cu") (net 16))
 (segment (start 168.96 97.12) (end 169 97.08) (width 0.2) (layer "F.Cu") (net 19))
 (segment (start 165 97.12) (end 168.96 97.12) (width 0.2) (layer "F.Cu") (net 19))
 (segment (start 132 102.2) (end 135.96 102.2) (width 0.2) (layer "F.Cu") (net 12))
 (segment (start 135.96 102.2) (end 136 102.16) (width 0.2) (layer "F.Cu") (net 12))
 (segment (start 135.96 99.66) (end 136 99.62) (width 0.2) (layer "F.Cu") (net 13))
 (segment (start 132 99.66) (end 135.96 99.66) (width 0.2) (layer "F.Cu") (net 13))
 (segment (start 132 92.04) (end 135.96 92.04) (width 0.2) (layer "F.Cu") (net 10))
 (segment (start 135.96 92.04) (end 136 92) (width 0.2) (layer "F.Cu") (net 10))
 (segment (start 132 94.58) (end 135.96 94.58) (width 0.2) (layer "F.Cu") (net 9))
 (segment (start 135.96 94.58) (end 136 94.54) (width 0.2) (layer "F.Cu") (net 9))
 (segment (start 178.11 129) (end 188.61 118.5) (width 0.2) (layer "B.Cu") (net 31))
 (segment (start 120.48 129) (end 178.11 129) (width 0.2) (layer "B.Cu") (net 31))
 (segment (start 118.24 131.24) (end 120.48 129) (width 0.2) (layer "B.Cu") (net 31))
 (segment (start 176.57 128) (end 186.07 118.5) (width 0.2) (layer "B.Cu") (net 30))
 (segment (start 118.94 128) (end 176.57 128) (width 0.2) (layer "B.Cu") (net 30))
 (segment (start 115.7 131.24) (end 118.94 128) (width 0.2) (layer "B.Cu") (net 30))
 (segment (start 116.801 127.599) (end 113.16 131.24) (width 0.2) (layer "B.Cu") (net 29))
 (segment (start 160.16 118.5) (end 151.061 127.599) (width 0.2) (layer "B.Cu") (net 29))
 (segment (start 151.061 127.599) (end 116.801 127.599) (width 0.2) (layer "B.Cu") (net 29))
 (segment (start 114.662 127.198) (end 110.62 131.24) (width 0.2) (layer "B.Cu") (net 28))
 (segment (start 148.922 127.198) (end 114.662 127.198) (width 0.2) (layer "B.Cu") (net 28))
 (segment (start 157.62 118.5) (end 148.922 127.198) (width 0.2) (layer "B.Cu") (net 28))
 (segment (start 105.54 131.24) (end 108.3 134) (width 0.2) (layer "B.Cu") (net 2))
 (segment (start 130.75 134) (end 133.5 131.25) (width 0.2) (layer "B.Cu") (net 2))
 (segment (start 108.3 134) (end 130.75 134) (width 0.2) (layer "B.Cu") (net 2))
 (segment (start 147.81 147) (end 147.81 131.06) (width 0.2) (layer "F.Cu") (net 4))
 (segment (start 153 147) (end 147.81 147) (width 0.2) (layer "F.Cu") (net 4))
 (segment (start 147.81 131.06) (end 133.5 116.75) (width 0.2) (layer "F.Cu") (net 4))
 (segment (start 109.143 132.303) (end 127.447 132.303) (width 0.2) (layer "B.Cu") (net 1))
 (segment (start 127.447 132.303) (end 128.5 131.25) (width 0.2) (layer "B.Cu") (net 1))
 (segment (start 108.08 131.24) (end 109.143 132.303) (width 0.2) (layer "B.Cu") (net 1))
 (segment (start 113.16 116) (end 113.16 109.78) (width 0.2) (layer "B.Cu") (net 8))
 (segment (start 113.16 109.78) (end 103 99.62) (width 0.2) (layer "B.Cu") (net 8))
 (segment (start 110.62 116) (end 110.62 109.78) (width 0.2) (layer "B.Cu") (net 7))
 (segment (start 110.62 109.78) (end 103 102.16) (width 0.2) (layer "B.Cu") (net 7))
 (segment (start 115.7 109.78) (end 103 97.08) (width 0.2) (layer "B.Cu") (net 6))
 (segment (start 115.7 116) (end 115.7 109.78) (width 0.2) (layer "B.Cu") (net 6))
 (segment (start 168.96 92.04) (end 169 92) (width 0.2) (layer "F.Cu") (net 18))
 (segment (start 165 92.04) (end 168.96 92.04) (width 0.2) (layer "F.Cu") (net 18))
 (segment (start 165 102.2) (end 168.96 102.2) (width 0.2) (layer "F.Cu") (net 20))
 (segment (start 168.96 102.2) (end 169 102.16) (width 0.2) (layer "F.Cu") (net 20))
 (segment (start 168.96 99.66) (end 169 99.62) (width 0.2) (layer "F.Cu") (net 21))
 (segment (start 165 99.66) (end 168.96 99.66) (width 0.2) (layer "F.Cu") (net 21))
 (segment (start 169 94.54) (end 165.04 94.54) (width 0.2) (layer "F.Cu") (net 17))
 (segment (start 168.96 94.58) (end 169 94.54) (width 0.2) (layer "F.Cu") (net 17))
 (segment (start 165.04 94.54) (end 165 94.58) (width 0.2) (layer "F.Cu") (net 17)))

